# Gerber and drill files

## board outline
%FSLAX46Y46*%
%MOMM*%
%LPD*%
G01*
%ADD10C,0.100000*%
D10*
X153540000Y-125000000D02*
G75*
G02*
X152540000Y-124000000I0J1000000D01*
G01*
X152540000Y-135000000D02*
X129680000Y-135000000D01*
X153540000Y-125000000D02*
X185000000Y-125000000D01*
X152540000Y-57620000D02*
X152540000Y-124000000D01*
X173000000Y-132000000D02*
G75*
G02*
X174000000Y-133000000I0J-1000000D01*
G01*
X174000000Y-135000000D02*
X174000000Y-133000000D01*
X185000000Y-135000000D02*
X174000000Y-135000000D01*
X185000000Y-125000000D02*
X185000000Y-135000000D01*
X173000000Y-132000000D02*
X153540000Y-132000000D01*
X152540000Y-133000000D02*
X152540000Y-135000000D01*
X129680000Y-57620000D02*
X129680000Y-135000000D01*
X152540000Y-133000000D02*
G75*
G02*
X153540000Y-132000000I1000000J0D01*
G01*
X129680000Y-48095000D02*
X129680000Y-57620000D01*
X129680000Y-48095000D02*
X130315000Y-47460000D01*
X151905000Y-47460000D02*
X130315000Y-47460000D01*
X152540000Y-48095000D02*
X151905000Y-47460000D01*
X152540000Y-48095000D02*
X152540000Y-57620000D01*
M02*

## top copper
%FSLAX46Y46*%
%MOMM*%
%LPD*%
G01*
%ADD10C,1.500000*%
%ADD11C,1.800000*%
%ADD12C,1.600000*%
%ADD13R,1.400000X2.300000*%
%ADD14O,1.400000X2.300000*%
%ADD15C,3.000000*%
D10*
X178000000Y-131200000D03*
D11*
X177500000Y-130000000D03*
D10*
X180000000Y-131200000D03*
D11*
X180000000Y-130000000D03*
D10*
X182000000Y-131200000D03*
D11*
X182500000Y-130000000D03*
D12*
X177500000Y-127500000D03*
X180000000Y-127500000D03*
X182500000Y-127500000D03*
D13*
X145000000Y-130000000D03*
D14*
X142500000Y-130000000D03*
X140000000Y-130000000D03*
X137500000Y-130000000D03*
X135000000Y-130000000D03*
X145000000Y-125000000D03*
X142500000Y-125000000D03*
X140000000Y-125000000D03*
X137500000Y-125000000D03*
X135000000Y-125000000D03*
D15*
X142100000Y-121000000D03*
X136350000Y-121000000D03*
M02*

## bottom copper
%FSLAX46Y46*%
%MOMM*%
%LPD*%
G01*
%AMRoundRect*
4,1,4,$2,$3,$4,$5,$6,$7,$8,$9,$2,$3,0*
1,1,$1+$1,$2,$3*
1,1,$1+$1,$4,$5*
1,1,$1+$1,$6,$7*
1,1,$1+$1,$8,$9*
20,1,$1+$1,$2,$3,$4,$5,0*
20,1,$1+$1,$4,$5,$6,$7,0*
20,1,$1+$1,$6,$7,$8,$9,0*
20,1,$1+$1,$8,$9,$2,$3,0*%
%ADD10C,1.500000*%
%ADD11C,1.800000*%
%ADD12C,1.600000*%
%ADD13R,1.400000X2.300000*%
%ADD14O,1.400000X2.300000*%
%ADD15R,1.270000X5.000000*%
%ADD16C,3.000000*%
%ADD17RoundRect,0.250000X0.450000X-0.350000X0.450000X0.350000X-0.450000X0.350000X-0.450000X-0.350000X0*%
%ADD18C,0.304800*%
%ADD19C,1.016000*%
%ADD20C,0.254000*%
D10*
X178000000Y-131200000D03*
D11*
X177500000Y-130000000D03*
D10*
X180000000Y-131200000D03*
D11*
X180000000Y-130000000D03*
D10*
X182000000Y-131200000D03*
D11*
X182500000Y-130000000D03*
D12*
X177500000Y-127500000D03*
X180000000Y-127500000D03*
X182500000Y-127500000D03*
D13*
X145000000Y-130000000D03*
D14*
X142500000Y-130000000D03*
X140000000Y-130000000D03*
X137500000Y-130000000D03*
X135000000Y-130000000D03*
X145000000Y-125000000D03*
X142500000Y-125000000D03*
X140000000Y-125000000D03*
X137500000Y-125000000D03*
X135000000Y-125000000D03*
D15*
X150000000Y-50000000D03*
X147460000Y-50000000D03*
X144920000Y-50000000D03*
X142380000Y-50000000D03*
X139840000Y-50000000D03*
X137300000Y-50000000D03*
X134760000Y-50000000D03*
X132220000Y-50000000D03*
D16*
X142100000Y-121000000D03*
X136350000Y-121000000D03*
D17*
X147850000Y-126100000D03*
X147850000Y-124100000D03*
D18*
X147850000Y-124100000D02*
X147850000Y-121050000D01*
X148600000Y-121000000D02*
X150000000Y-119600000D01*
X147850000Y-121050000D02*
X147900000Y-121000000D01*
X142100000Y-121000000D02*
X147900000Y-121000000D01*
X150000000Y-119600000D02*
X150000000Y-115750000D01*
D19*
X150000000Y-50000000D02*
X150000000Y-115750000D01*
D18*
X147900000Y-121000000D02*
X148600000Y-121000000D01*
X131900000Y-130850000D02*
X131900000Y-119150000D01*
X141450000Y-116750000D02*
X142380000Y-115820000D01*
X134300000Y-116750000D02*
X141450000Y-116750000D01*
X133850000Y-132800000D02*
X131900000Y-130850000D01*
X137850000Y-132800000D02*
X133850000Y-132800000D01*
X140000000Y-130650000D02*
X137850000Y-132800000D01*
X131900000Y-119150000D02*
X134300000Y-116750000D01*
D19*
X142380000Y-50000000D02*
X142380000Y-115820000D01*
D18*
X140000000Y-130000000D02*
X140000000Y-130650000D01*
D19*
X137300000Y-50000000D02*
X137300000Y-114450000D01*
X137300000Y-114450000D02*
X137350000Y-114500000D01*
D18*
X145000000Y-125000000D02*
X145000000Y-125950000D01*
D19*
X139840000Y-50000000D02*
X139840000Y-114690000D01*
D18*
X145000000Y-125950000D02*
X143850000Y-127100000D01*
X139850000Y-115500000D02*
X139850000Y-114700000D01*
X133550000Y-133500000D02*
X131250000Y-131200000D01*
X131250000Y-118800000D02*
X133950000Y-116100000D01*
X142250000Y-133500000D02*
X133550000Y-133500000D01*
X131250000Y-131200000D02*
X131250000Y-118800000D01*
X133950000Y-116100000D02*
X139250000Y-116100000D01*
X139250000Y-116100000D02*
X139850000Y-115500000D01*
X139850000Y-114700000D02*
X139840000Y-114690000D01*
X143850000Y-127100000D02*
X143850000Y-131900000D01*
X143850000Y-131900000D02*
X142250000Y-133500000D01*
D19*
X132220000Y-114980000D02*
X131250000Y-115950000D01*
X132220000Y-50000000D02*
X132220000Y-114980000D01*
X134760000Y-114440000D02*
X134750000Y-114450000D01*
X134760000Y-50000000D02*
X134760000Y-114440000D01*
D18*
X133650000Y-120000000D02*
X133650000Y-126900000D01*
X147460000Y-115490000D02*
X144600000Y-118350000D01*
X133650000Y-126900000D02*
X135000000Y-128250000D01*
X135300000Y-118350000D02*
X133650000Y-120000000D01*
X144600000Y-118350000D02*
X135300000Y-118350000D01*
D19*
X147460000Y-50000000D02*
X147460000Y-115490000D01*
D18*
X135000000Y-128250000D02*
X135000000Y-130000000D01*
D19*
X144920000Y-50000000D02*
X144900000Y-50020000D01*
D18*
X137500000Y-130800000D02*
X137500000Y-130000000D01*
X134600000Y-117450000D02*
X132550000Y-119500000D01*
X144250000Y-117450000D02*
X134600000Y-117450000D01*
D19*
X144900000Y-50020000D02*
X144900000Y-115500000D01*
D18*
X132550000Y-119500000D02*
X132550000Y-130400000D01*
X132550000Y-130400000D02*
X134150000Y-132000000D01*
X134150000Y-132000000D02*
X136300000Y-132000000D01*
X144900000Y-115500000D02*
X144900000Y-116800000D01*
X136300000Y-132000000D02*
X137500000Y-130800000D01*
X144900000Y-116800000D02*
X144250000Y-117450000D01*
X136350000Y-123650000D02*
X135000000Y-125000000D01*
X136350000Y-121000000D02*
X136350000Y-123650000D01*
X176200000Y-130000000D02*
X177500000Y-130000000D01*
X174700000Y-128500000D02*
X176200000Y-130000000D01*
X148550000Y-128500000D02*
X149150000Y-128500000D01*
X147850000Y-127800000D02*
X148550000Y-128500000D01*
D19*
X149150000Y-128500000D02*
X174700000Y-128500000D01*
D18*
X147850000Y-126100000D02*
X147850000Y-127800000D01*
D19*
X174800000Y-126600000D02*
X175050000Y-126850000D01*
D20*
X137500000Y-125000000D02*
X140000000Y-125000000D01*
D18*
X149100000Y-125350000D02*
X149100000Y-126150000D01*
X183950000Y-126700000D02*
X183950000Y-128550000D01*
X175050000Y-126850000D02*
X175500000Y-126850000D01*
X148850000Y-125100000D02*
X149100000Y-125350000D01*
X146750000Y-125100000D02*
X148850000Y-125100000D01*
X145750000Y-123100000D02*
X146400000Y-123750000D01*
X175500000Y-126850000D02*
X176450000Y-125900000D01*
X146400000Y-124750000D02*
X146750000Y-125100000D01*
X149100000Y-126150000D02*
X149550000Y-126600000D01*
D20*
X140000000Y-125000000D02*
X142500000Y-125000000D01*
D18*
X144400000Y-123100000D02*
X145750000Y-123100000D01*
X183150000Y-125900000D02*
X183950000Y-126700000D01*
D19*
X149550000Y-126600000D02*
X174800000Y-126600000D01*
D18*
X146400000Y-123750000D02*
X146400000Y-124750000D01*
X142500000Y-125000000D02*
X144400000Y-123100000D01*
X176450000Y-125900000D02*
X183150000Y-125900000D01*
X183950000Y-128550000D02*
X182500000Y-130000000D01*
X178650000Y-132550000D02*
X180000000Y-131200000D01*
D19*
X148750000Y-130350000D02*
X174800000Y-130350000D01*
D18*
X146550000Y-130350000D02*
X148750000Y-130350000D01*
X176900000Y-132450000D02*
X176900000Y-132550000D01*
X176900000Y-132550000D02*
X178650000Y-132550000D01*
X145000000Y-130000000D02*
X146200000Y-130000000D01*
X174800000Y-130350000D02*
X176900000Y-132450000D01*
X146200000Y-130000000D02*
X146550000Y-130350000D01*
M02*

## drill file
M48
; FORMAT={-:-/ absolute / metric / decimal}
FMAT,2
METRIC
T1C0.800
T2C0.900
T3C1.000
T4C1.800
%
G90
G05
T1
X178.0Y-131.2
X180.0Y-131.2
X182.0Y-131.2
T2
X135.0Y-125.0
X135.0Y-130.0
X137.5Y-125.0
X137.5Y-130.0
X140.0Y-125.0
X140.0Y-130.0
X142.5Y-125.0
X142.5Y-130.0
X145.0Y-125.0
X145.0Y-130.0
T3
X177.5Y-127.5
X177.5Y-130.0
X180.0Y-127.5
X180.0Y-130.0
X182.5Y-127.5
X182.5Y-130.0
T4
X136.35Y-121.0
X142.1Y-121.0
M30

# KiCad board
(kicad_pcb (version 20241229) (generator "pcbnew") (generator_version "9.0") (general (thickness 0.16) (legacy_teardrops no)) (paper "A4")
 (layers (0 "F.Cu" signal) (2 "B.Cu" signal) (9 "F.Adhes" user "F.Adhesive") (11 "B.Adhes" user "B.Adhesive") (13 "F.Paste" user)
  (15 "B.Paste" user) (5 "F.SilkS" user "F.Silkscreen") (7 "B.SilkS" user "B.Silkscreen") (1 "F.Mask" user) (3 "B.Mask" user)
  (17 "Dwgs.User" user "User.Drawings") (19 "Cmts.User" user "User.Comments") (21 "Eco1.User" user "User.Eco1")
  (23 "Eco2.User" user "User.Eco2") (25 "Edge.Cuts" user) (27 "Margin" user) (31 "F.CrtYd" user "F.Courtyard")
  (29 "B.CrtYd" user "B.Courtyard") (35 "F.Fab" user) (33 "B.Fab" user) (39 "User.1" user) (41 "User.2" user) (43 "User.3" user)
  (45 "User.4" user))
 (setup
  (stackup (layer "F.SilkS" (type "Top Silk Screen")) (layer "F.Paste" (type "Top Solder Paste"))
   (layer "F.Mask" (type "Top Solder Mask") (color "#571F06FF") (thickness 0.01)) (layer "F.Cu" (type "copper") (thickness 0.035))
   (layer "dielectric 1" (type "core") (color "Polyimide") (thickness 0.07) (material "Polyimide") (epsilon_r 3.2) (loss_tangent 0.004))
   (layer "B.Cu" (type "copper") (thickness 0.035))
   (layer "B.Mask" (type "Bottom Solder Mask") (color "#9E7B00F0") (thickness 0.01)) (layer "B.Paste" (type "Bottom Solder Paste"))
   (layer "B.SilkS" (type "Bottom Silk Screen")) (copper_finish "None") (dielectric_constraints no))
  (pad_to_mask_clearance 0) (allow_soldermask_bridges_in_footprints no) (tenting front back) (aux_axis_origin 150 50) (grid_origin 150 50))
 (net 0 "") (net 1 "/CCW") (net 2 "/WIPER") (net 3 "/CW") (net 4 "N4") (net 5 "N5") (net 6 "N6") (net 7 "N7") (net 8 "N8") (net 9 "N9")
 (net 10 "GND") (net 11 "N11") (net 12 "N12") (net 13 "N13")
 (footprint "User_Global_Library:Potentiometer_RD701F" (layer "F.Cu") (at 180 131.2 90)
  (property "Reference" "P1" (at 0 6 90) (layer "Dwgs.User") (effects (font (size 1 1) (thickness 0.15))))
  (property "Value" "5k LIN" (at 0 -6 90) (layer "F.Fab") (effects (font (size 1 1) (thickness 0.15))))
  (pad "1" thru_hole circle (at 0 -2 90) (size 1.5 1.5) (drill 0.8) (layers "*.Cu" "*.Mask") (remove_unused_layers no) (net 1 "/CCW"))
  (pad "1" thru_hole circle (at 1.2 -2.5 90) (size 1.8 1.8) (drill 1) (layers "*.Cu" "*.Mask") (remove_unused_layers no) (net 1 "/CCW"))
  (pad "2" thru_hole circle (at 0 0 90) (size 1.5 1.5) (drill 0.8) (layers "*.Cu" "*.Mask") (remove_unused_layers no) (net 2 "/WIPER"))
  (pad "2" thru_hole circle (at 1.2 0 90) (size 1.8 1.8) (drill 1) (layers "*.Cu" "*.Mask") (remove_unused_layers no) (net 2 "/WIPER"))
  (pad "3" thru_hole circle (at 0 2 90) (size 1.5 1.5) (drill 0.8) (layers "*.Cu" "*.Mask") (remove_unused_layers no) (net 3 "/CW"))
  (pad "3" thru_hole circle (at 1.2 2.5 90) (size 1.8 1.8) (drill 1) (layers "*.Cu" "*.Mask") (remove_unused_layers no) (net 3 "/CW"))
  (pad "MP" thru_hole circle (at 3.7 -2.5 90) (size 1.6 1.6) (drill 1) (layers "*.Cu" "*.Mask") (remove_unused_layers no))
  (pad "MP" thru_hole circle (at 3.7 0 90) (size 1.6 1.6) (drill 1) (layers "*.Cu" "*.Mask") (remove_unused_layers no))
  (pad "MP" thru_hole circle (at 3.7 2.5 90) (size 1.6 1.6) (drill 1) (layers "*.Cu" "*.Mask") (remove_unused_layers no)))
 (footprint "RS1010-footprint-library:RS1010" (layer "F.Cu") (at 140 135 -90)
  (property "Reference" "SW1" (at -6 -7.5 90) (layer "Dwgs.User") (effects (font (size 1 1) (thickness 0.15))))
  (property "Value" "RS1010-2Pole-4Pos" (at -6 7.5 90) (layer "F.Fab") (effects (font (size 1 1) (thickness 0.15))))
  (pad "1" thru_hole rect (at -5 -5 270) (size 2.3 1.4) (drill 0.9) (layers "*.Cu" "*.Mask") (remove_unused_layers no) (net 2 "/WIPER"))
  (pad "2" thru_hole oval (at -5 -2.5 270) (size 2.3 1.4) (drill 0.9) (layers "*.Cu" "*.Mask") (remove_unused_layers no) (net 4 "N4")
   (thermal_bridge_angle 45))
  (pad "3" thru_hole oval (at -5 0 270) (size 2.3 1.4) (drill 0.9) (layers "*.Cu" "*.Mask") (remove_unused_layers no) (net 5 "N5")
   (thermal_bridge_angle 45))
  (pad "4" thru_hole oval (at -5 2.5 270) (size 2.3 1.4) (drill 0.9) (layers "*.Cu" "*.Mask") (remove_unused_layers no) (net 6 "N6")
   (thermal_bridge_angle 45))
  (pad "5" thru_hole oval (at -5 5 270) (size 2.3 1.4) (drill 0.9) (layers "*.Cu" "*.Mask") (remove_unused_layers no) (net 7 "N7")
   (thermal_bridge_angle 45))
  (pad "6" thru_hole oval (at -10 -5 270) (size 2.3 1.4) (drill 0.9) (layers "*.Cu" "*.Mask") (remove_unused_layers no) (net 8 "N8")
   (thermal_bridge_angle 45))
  (pad "7" thru_hole oval (at -10 -2.5 270) (size 2.3 1.4) (drill 0.9) (layers "*.Cu" "*.Mask") (remove_unused_layers no) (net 3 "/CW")
   (thermal_bridge_angle 45))
  (pad "8" thru_hole oval (at -10 0 270) (size 2.3 1.4) (drill 0.9) (layers "*.Cu" "*.Mask") (remove_unused_layers no) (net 3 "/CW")
   (thermal_bridge_angle 45))
  (pad "9" thru_hole oval (at -10 2.5 270) (size 2.3 1.4) (drill 0.9) (layers "*.Cu" "*.Mask") (remove_unused_layers no) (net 3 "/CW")
   (thermal_bridge_angle 45))
  (pad "10" thru_hole oval (at -10 5 270) (size 2.3 1.4) (drill 0.9) (layers "*.Cu" "*.Mask") (remove_unused_layers no) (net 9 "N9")
   (thermal_bridge_angle 45)))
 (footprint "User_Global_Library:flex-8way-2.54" (layer "B.Cu") (at 150 50 90)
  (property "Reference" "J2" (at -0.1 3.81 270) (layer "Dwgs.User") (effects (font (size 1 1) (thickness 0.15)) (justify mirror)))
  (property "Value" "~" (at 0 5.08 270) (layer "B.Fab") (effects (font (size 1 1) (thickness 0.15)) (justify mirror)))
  (fp_line (start 1.905 -20.32) (end -7.62 -20.32) (stroke (width 0.1) (type default)) (layer "Edge.Cuts"))
  (fp_line (start 1.905 -20.32) (end 2.54 -19.685) (stroke (width 0.1) (type default)) (layer "Edge.Cuts"))
  (fp_line (start 2.54 1.905) (end 2.54 -19.685) (stroke (width 0.1) (type default)) (layer "Edge.Cuts"))
  (fp_line (start 1.905 2.54) (end 2.54 1.905) (stroke (width 0.1) (type default)) (layer "Edge.Cuts"))
  (fp_line (start 1.905 2.54) (end -7.62 2.54) (stroke (width 0.1) (type default)) (layer "Edge.Cuts"))
  (pad "1" smd rect (at 0 0 90) (size 5 1.27) (layers "B.Cu" "B.Mask" "B.Paste") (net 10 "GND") (thermal_bridge_angle 45))
  (pad "2" smd rect (at 0 -2.54 90) (size 5 1.27) (layers "B.Cu" "B.Mask" "B.Paste") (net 7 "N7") (thermal_bridge_angle 45))
  (pad "3" smd rect (at 0 -5.08 90) (size 5 1.27) (layers "B.Cu" "B.Mask" "B.Paste") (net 6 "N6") (thermal_bridge_angle 45))
  (pad "4" smd rect (at 0 -7.62 90) (size 5 1.27) (layers "B.Cu" "B.Mask" "B.Paste") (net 5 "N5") (thermal_bridge_angle 45))
  (pad "5" smd rect (at 0 -10.16 90) (size 5 1.27) (layers "B.Cu" "B.Mask" "B.Paste") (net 8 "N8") (thermal_bridge_angle 45))
  (pad "6" smd rect (at 0 -12.7 90) (size 5 1.27) (layers "B.Cu" "B.Mask" "B.Paste") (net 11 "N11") (thermal_bridge_angle 45))
  (pad "7" smd rect (at 0 -15.24 90) (size 5 1.27) (layers "B.Cu" "B.Mask" "B.Paste") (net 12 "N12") (thermal_bridge_angle 45))
  (pad "8" smd rect (at 0 -17.78 90) (size 5 1.27) (layers "B.Cu" "B.Mask" "B.Paste") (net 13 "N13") (thermal_bridge_angle 45)))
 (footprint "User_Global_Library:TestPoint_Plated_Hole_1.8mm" (layer "B.Cu") (at 142.1 121)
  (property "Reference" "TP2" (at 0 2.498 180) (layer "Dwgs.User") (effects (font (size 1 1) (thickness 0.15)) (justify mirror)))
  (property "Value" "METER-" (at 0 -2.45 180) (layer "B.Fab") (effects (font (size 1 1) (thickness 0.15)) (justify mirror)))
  (pad "1" thru_hole circle (at 0 0) (size 3 3) (drill 1.8) (layers "*.Cu" "*.Mask") (remove_unused_layers no) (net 10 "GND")))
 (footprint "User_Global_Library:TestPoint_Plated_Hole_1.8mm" (layer "B.Cu") (at 136.35 121)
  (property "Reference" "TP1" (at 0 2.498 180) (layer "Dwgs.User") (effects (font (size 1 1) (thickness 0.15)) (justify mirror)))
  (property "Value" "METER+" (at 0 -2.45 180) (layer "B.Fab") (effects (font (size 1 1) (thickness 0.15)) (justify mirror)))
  (pad "1" thru_hole circle (at 0 0) (size 3 3) (drill 1.8) (layers "*.Cu" "*.Mask") (remove_unused_layers no) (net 9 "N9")))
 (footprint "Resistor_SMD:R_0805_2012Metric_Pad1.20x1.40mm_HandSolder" (layer "B.Cu") (at 147.85 125.1 90)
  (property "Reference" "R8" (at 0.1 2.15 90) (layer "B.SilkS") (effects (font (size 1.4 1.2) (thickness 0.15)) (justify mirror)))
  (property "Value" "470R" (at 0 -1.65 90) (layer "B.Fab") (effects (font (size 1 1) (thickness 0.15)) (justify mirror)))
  (pad "1" smd roundrect (at -1 0 90) (size 1.2 1.4) (layers "B.Cu" "B.Mask" "B.Paste") (roundrect_rratio 0.208333) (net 1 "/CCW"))
  (pad "2" smd roundrect (at 1 0 90) (size 1.2 1.4) (layers "B.Cu" "B.Mask" "B.Paste") (roundrect_rratio 0.208333) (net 10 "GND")))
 (gr_arc (start 153.54 125) (mid 152.832893 124.707107) (end 152.54 124) (stroke (width 0.1) (type default)) (layer "Edge.Cuts"))
 (gr_line (start 152.54 135) (end 129.68 135) (stroke (width 0.1) (type default)) (layer "Edge.Cuts"))
 (gr_line (start 153.54 125) (end 185 125) (stroke (width 0.1) (type default)) (layer "Edge.Cuts"))
 (gr_line (start 152.54 57.62) (end 152.54 124) (stroke (width 0.1) (type default)) (layer "Edge.Cuts"))
 (gr_arc (start 173 132) (mid 173.707107 132.292893) (end 174 133) (stroke (width 0.1) (type default)) (layer "Edge.Cuts"))
 (gr_line (start 174 135) (end 174 133) (stroke (width 0.1) (type default)) (layer "Edge.Cuts"))
 (gr_line (start 185 135) (end 174 135) (stroke (width 0.1) (type default)) (layer "Edge.Cuts"))
 (gr_line (start 185 125) (end 185 135) (stroke (width 0.1) (type default)) (layer "Edge.Cuts"))
 (gr_line (start 173 132) (end 153.54 132) (stroke (width 0.1) (type default)) (layer "Edge.Cuts"))
 (gr_line (start 152.54 133) (end 152.54 135) (stroke (width 0.1) (type default)) (layer "Edge.Cuts"))
 (gr_line (start 129.68 57.62) (end 129.68 135) (stroke (width 0.1) (type default)) (layer "Edge.Cuts"))
 (gr_arc (start 152.54 133) (mid 152.832893 132.292893) (end 153.54 132) (stroke (width 0.1) (type default)) (layer "Edge.Cuts"))
 (segment (start 147.85 124.1) (end 147.85 121.05) (width 0.3048) (layer "B.Cu") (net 10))
 (segment (start 148.6 121) (end 150 119.6) (width 0.3048) (layer "B.Cu") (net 10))
 (segment (start 147.85 121.05) (end 147.9 121) (width 0.3048) (layer "B.Cu") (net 10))
 (segment (start 142.1 121) (end 147.9 121) (width 0.3048) (layer "B.Cu") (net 10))
 (segment (start 150 119.6) (end 150 115.75) (width 0.3048) (layer "B.Cu") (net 10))
 (segment (start 150 50) (end 150 115.75) (width 1.016) (layer "B.Cu") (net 10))
 (segment (start 147.9 121) (end 148.6 121) (width 0.3048) (layer "B.Cu") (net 10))
 (segment (start 131.9 130.85) (end 131.9 119.15) (width 0.3048) (layer "B.Cu") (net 5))
 (segment (start 141.45 116.75) (end 142.38 115.82) (width 0.3048) (layer "B.Cu") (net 5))
 (segment (start 134.3 116.75) (end 141.45 116.75) (width 0.3048) (layer "B.Cu") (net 5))
 (segment (start 133.85 132.8) (end 131.9 130.85) (width 0.3048) (layer "B.Cu") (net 5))
 (segment (start 137.85 132.8) (end 133.85 132.8) (width 0.3048) (layer "B.Cu") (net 5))
 (segment (start 140 130.65) (end 137.85 132.8) (width 0.3048) (layer "B.Cu") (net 5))
 (segment (start 131.9 119.15) (end 134.3 116.75) (width 0.3048) (layer "B.Cu") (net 5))
 (segment (start 142.38 50) (end 142.38 115.82) (width 1.016) (layer "B.Cu") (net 5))
 (segment (start 140 130) (end 140 130.65) (width 0.3048) (layer "B.Cu") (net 5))
 (segment (start 137.3 50) (end 137.3 114.45) (width 1.016) (layer "B.Cu") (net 11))
 (segment (start 137.3 114.45) (end 137.35 114.5) (width 1.016) (layer "B.Cu") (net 11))
 (segment (start 145 125) (end 145 125.95) (width 0.3048) (layer "B.Cu") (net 8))
 (segment (start 139.84 50) (end 139.84 114.69) (width 1.016) (layer "B.Cu") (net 8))
 (segment (start 145 125.95) (end 143.85 127.1) (width 0.3048) (layer "B.Cu") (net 8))
 (segment (start 139.85 115.5) (end 139.85 114.7) (width 0.3048) (layer "B.Cu") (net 8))
 (segment (start 133.55 133.5) (end 131.25 131.2) (width 0.3048) (layer "B.Cu") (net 8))
 (segment (start 131.25 118.8) (end 133.95 116.1) (width 0.3048) (layer "B.Cu") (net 8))
 (segment (start 142.25 133.5) (end 133.55 133.5) (width 0.3048) (layer "B.Cu") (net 8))
 (segment (start 131.25 131.2) (end 131.25 118.8) (width 0.3048) (layer "B.Cu") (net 8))
 (segment (start 133.95 116.1) (end 139.25 116.1) (width 0.3048) (layer "B.Cu") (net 8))
 (segment (start 139.25 116.1) (end 139.85 115.5) (width 0.3048) (layer "B.Cu") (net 8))
 (segment (start 139.85 114.7) (end 139.84 114.69) (width 0.3048) (layer "B.Cu") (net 8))
 (segment (start 143.85 127.1) (end 143.85 131.9) (width 0.3048) (layer "B.Cu") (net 8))
 (segment (start 143.85 131.9) (end 142.25 133.5) (width 0.3048) (layer "B.Cu") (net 8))
 (segment (start 132.22 114.98) (end 131.25 115.95) (width 1.016) (layer "B.Cu") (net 13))
 (segment (start 132.22 50) (end 132.22 114.98) (width 1.016) (layer "B.Cu") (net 13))
 (segment (start 134.76 114.44) (end 134.75 114.45) (width 1.016) (layer "B.Cu") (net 12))
 (segment (start 134.76 50) (end 134.76 114.44) (width 1.016) (layer "B.Cu") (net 12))
 (segment (start 133.65 120) (end 133.65 126.9) (width 0.3048) (layer "B.Cu") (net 7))
 (segment (start 147.46 115.49) (end 144.6 118.35) (width 0.3048) (layer "B.Cu") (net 7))
 (segment (start 133.65 126.9) (end 135 128.25) (width 0.3048) (layer "B.Cu") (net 7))
 (segment (start 135.3 118.35) (end 133.65 120) (width 0.3048) (layer "B.Cu") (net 7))
 (segment (start 144.6 118.35) (end 135.3 118.35) (width 0.3048) (layer "B.Cu") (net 7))
 (segment (start 147.46 50) (end 147.46 115.49) (width 1.016) (layer "B.Cu") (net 7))
 (segment (start 135 128.25) (end 135 130) (width 0.3048) (layer "B.Cu") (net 7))
 (segment (start 144.92 50) (end 144.9 50.02) (width 1.016) (layer "B.Cu") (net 6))
 (segment (start 137.5 130.8) (end 137.5 130) (width 0.3048) (layer "B.Cu") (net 6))
 (segment (start 134.6 117.45) (end 132.55 119.5) (width 0.3048) (layer "B.Cu") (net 6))
 (segment (start 144.25 117.45) (end 134.6 117.45) (width 0.3048) (layer "B.Cu") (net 6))
 (segment (start 144.9 50.02) (end 144.9 115.5) (width 1.016) (layer "B.Cu") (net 6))
 (segment (start 132.55 119.5) (end 132.55 130.4) (width 0.3048) (layer "B.Cu") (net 6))
 (segment (start 132.55 130.4) (end 134.15 132) (width 0.3048) (layer "B.Cu") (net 6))
 (segment (start 134.15 132) (end 136.3 132) (width 0.3048) (layer "B.Cu") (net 6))
 (segment (start 144.9 115.5) (end 144.9 116.8) (width 0.3048) (layer "B.Cu") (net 6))
 (segment (start 136.3 132) (end 137.5 130.8) (width 0.3048) (layer "B.Cu") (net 6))
 (segment (start 144.9 116.8) (end 144.25 117.45) (width 0.3048) (layer "B.Cu") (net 6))
 (segment (start 136.35 123.65) (end 135 125) (width 0.3048) (layer "B.Cu") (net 9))
 (segment (start 136.35 121) (end 136.35 123.65) (width 0.3048) (layer "B.Cu") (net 9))
 (segment (start 176.2 130) (end 177.5 130) (width 0.3048) (layer "B.Cu") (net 1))
 (segment (start 174.7 128.5) (end 176.2 130) (width 0.3048) (layer "B.Cu") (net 1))
 (segment (start 148.55 128.5) (end 149.15 128.5) (width 0.3048) (layer "B.Cu") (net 1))
 (segment (start 147.85 127.8) (end 148.55 128.5) (width 0.3048) (layer "B.Cu") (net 1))
 (segment (start 149.15 128.5) (end 174.7 128.5) (width 1.016) (layer "B.Cu") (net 1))
 (segment (start 147.85 126.1) (end 147.85 127.8) (width 0.3048) (layer "B.Cu") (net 1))
 (segment (start 174.8 126.6) (end 175.05 126.85) (width 1.016) (layer "B.Cu") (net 3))
 (segment (start 137.5 125) (end 140 125) (width 0.254) (layer "B.Cu") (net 3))
 (segment (start 149.1 125.35) (end 149.1 126.15) (width 0.3048) (layer "B.Cu") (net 3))
 (segment (start 183.95 126.7) (end 183.95 128.55) (width 0.3048) (layer "B.Cu") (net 3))
 (segment (start 175.05 126.85) (end 175.5 126.85) (width 0.3048) (layer "B.Cu") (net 3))
 (segment (start 148.85 125.1) (end 149.1 125.35) (width 0.3048) (layer "B.Cu") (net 3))
 (segment (start 146.75 125.1) (end 148.85 125.1) (width 0.3048) (layer "B.Cu") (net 3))
 (segment (start 145.75 123.1) (end 146.4 123.75) (width 0.3048) (layer "B.Cu") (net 3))
 (segment (start 175.5 126.85) (end 176.45 125.9) (width 0.3048) (layer "B.Cu") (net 3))
 (segment (start 146.4 124.75) (end 146.75 125.1) (width 0.3048) (layer "B.Cu") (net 3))
 (segment (start 149.1 126.15) (end 149.55 126.6) (width 0.3048) (layer "B.Cu") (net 3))
 (segment (start 140 125) (end 142.5 125) (width 0.254) (layer "B.Cu") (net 3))
 (segment (start 144.4 123.1) (end 145.75 123.1) (width 0.3048) (layer "B.Cu") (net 3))
 (segment (start 183.15 125.9) (end 183.95 126.7) (width 0.3048) (layer "B.Cu") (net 3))
 (segment (start 149.55 126.6) (end 174.8 126.6) (width 1.016) (layer "B.Cu") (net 3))
 (segment (start 146.4 123.75) (end 146.4 124.75) (width 0.3048) (layer "B.Cu") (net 3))
 (segment (start 142.5 125) (end 144.4 123.1) (width 0.3048) (layer "B.Cu") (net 3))
 (segment (start 176.45 125.9) (end 183.15 125.9) (width 0.3048) (layer "B.Cu") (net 3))
 (segment (start 183.95 128.55) (end 182.5 130) (width 0.3048) (layer "B.Cu") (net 3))
 (segment (start 178.65 132.55) (end 180 131.2) (width 0.3048) (layer "B.Cu") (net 2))
 (segment (start 148.75 130.35) (end 174.8 130.35) (width 1.016) (layer "B.Cu") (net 2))
 (segment (start 146.55 130.35) (end 148.75 130.35) (width 0.3048) (layer "B.Cu") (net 2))
 (segment (start 176.9 132.45) (end 176.9 132.55) (width 0.3048) (layer "B.Cu") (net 2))
 (segment (start 176.9 132.55) (end 178.65 132.55) (width 0.3048) (layer "B.Cu") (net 2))
 (segment (start 145 130) (end 146.2 130) (width 0.3048) (layer "B.Cu") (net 2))
 (segment (start 174.8 130.35) (end 176.9 132.45) (width 0.3048) (layer "B.Cu") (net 2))
 (segment (start 146.2 130) (end 146.55 130.35) (width 0.3048) (layer "B.Cu") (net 2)))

